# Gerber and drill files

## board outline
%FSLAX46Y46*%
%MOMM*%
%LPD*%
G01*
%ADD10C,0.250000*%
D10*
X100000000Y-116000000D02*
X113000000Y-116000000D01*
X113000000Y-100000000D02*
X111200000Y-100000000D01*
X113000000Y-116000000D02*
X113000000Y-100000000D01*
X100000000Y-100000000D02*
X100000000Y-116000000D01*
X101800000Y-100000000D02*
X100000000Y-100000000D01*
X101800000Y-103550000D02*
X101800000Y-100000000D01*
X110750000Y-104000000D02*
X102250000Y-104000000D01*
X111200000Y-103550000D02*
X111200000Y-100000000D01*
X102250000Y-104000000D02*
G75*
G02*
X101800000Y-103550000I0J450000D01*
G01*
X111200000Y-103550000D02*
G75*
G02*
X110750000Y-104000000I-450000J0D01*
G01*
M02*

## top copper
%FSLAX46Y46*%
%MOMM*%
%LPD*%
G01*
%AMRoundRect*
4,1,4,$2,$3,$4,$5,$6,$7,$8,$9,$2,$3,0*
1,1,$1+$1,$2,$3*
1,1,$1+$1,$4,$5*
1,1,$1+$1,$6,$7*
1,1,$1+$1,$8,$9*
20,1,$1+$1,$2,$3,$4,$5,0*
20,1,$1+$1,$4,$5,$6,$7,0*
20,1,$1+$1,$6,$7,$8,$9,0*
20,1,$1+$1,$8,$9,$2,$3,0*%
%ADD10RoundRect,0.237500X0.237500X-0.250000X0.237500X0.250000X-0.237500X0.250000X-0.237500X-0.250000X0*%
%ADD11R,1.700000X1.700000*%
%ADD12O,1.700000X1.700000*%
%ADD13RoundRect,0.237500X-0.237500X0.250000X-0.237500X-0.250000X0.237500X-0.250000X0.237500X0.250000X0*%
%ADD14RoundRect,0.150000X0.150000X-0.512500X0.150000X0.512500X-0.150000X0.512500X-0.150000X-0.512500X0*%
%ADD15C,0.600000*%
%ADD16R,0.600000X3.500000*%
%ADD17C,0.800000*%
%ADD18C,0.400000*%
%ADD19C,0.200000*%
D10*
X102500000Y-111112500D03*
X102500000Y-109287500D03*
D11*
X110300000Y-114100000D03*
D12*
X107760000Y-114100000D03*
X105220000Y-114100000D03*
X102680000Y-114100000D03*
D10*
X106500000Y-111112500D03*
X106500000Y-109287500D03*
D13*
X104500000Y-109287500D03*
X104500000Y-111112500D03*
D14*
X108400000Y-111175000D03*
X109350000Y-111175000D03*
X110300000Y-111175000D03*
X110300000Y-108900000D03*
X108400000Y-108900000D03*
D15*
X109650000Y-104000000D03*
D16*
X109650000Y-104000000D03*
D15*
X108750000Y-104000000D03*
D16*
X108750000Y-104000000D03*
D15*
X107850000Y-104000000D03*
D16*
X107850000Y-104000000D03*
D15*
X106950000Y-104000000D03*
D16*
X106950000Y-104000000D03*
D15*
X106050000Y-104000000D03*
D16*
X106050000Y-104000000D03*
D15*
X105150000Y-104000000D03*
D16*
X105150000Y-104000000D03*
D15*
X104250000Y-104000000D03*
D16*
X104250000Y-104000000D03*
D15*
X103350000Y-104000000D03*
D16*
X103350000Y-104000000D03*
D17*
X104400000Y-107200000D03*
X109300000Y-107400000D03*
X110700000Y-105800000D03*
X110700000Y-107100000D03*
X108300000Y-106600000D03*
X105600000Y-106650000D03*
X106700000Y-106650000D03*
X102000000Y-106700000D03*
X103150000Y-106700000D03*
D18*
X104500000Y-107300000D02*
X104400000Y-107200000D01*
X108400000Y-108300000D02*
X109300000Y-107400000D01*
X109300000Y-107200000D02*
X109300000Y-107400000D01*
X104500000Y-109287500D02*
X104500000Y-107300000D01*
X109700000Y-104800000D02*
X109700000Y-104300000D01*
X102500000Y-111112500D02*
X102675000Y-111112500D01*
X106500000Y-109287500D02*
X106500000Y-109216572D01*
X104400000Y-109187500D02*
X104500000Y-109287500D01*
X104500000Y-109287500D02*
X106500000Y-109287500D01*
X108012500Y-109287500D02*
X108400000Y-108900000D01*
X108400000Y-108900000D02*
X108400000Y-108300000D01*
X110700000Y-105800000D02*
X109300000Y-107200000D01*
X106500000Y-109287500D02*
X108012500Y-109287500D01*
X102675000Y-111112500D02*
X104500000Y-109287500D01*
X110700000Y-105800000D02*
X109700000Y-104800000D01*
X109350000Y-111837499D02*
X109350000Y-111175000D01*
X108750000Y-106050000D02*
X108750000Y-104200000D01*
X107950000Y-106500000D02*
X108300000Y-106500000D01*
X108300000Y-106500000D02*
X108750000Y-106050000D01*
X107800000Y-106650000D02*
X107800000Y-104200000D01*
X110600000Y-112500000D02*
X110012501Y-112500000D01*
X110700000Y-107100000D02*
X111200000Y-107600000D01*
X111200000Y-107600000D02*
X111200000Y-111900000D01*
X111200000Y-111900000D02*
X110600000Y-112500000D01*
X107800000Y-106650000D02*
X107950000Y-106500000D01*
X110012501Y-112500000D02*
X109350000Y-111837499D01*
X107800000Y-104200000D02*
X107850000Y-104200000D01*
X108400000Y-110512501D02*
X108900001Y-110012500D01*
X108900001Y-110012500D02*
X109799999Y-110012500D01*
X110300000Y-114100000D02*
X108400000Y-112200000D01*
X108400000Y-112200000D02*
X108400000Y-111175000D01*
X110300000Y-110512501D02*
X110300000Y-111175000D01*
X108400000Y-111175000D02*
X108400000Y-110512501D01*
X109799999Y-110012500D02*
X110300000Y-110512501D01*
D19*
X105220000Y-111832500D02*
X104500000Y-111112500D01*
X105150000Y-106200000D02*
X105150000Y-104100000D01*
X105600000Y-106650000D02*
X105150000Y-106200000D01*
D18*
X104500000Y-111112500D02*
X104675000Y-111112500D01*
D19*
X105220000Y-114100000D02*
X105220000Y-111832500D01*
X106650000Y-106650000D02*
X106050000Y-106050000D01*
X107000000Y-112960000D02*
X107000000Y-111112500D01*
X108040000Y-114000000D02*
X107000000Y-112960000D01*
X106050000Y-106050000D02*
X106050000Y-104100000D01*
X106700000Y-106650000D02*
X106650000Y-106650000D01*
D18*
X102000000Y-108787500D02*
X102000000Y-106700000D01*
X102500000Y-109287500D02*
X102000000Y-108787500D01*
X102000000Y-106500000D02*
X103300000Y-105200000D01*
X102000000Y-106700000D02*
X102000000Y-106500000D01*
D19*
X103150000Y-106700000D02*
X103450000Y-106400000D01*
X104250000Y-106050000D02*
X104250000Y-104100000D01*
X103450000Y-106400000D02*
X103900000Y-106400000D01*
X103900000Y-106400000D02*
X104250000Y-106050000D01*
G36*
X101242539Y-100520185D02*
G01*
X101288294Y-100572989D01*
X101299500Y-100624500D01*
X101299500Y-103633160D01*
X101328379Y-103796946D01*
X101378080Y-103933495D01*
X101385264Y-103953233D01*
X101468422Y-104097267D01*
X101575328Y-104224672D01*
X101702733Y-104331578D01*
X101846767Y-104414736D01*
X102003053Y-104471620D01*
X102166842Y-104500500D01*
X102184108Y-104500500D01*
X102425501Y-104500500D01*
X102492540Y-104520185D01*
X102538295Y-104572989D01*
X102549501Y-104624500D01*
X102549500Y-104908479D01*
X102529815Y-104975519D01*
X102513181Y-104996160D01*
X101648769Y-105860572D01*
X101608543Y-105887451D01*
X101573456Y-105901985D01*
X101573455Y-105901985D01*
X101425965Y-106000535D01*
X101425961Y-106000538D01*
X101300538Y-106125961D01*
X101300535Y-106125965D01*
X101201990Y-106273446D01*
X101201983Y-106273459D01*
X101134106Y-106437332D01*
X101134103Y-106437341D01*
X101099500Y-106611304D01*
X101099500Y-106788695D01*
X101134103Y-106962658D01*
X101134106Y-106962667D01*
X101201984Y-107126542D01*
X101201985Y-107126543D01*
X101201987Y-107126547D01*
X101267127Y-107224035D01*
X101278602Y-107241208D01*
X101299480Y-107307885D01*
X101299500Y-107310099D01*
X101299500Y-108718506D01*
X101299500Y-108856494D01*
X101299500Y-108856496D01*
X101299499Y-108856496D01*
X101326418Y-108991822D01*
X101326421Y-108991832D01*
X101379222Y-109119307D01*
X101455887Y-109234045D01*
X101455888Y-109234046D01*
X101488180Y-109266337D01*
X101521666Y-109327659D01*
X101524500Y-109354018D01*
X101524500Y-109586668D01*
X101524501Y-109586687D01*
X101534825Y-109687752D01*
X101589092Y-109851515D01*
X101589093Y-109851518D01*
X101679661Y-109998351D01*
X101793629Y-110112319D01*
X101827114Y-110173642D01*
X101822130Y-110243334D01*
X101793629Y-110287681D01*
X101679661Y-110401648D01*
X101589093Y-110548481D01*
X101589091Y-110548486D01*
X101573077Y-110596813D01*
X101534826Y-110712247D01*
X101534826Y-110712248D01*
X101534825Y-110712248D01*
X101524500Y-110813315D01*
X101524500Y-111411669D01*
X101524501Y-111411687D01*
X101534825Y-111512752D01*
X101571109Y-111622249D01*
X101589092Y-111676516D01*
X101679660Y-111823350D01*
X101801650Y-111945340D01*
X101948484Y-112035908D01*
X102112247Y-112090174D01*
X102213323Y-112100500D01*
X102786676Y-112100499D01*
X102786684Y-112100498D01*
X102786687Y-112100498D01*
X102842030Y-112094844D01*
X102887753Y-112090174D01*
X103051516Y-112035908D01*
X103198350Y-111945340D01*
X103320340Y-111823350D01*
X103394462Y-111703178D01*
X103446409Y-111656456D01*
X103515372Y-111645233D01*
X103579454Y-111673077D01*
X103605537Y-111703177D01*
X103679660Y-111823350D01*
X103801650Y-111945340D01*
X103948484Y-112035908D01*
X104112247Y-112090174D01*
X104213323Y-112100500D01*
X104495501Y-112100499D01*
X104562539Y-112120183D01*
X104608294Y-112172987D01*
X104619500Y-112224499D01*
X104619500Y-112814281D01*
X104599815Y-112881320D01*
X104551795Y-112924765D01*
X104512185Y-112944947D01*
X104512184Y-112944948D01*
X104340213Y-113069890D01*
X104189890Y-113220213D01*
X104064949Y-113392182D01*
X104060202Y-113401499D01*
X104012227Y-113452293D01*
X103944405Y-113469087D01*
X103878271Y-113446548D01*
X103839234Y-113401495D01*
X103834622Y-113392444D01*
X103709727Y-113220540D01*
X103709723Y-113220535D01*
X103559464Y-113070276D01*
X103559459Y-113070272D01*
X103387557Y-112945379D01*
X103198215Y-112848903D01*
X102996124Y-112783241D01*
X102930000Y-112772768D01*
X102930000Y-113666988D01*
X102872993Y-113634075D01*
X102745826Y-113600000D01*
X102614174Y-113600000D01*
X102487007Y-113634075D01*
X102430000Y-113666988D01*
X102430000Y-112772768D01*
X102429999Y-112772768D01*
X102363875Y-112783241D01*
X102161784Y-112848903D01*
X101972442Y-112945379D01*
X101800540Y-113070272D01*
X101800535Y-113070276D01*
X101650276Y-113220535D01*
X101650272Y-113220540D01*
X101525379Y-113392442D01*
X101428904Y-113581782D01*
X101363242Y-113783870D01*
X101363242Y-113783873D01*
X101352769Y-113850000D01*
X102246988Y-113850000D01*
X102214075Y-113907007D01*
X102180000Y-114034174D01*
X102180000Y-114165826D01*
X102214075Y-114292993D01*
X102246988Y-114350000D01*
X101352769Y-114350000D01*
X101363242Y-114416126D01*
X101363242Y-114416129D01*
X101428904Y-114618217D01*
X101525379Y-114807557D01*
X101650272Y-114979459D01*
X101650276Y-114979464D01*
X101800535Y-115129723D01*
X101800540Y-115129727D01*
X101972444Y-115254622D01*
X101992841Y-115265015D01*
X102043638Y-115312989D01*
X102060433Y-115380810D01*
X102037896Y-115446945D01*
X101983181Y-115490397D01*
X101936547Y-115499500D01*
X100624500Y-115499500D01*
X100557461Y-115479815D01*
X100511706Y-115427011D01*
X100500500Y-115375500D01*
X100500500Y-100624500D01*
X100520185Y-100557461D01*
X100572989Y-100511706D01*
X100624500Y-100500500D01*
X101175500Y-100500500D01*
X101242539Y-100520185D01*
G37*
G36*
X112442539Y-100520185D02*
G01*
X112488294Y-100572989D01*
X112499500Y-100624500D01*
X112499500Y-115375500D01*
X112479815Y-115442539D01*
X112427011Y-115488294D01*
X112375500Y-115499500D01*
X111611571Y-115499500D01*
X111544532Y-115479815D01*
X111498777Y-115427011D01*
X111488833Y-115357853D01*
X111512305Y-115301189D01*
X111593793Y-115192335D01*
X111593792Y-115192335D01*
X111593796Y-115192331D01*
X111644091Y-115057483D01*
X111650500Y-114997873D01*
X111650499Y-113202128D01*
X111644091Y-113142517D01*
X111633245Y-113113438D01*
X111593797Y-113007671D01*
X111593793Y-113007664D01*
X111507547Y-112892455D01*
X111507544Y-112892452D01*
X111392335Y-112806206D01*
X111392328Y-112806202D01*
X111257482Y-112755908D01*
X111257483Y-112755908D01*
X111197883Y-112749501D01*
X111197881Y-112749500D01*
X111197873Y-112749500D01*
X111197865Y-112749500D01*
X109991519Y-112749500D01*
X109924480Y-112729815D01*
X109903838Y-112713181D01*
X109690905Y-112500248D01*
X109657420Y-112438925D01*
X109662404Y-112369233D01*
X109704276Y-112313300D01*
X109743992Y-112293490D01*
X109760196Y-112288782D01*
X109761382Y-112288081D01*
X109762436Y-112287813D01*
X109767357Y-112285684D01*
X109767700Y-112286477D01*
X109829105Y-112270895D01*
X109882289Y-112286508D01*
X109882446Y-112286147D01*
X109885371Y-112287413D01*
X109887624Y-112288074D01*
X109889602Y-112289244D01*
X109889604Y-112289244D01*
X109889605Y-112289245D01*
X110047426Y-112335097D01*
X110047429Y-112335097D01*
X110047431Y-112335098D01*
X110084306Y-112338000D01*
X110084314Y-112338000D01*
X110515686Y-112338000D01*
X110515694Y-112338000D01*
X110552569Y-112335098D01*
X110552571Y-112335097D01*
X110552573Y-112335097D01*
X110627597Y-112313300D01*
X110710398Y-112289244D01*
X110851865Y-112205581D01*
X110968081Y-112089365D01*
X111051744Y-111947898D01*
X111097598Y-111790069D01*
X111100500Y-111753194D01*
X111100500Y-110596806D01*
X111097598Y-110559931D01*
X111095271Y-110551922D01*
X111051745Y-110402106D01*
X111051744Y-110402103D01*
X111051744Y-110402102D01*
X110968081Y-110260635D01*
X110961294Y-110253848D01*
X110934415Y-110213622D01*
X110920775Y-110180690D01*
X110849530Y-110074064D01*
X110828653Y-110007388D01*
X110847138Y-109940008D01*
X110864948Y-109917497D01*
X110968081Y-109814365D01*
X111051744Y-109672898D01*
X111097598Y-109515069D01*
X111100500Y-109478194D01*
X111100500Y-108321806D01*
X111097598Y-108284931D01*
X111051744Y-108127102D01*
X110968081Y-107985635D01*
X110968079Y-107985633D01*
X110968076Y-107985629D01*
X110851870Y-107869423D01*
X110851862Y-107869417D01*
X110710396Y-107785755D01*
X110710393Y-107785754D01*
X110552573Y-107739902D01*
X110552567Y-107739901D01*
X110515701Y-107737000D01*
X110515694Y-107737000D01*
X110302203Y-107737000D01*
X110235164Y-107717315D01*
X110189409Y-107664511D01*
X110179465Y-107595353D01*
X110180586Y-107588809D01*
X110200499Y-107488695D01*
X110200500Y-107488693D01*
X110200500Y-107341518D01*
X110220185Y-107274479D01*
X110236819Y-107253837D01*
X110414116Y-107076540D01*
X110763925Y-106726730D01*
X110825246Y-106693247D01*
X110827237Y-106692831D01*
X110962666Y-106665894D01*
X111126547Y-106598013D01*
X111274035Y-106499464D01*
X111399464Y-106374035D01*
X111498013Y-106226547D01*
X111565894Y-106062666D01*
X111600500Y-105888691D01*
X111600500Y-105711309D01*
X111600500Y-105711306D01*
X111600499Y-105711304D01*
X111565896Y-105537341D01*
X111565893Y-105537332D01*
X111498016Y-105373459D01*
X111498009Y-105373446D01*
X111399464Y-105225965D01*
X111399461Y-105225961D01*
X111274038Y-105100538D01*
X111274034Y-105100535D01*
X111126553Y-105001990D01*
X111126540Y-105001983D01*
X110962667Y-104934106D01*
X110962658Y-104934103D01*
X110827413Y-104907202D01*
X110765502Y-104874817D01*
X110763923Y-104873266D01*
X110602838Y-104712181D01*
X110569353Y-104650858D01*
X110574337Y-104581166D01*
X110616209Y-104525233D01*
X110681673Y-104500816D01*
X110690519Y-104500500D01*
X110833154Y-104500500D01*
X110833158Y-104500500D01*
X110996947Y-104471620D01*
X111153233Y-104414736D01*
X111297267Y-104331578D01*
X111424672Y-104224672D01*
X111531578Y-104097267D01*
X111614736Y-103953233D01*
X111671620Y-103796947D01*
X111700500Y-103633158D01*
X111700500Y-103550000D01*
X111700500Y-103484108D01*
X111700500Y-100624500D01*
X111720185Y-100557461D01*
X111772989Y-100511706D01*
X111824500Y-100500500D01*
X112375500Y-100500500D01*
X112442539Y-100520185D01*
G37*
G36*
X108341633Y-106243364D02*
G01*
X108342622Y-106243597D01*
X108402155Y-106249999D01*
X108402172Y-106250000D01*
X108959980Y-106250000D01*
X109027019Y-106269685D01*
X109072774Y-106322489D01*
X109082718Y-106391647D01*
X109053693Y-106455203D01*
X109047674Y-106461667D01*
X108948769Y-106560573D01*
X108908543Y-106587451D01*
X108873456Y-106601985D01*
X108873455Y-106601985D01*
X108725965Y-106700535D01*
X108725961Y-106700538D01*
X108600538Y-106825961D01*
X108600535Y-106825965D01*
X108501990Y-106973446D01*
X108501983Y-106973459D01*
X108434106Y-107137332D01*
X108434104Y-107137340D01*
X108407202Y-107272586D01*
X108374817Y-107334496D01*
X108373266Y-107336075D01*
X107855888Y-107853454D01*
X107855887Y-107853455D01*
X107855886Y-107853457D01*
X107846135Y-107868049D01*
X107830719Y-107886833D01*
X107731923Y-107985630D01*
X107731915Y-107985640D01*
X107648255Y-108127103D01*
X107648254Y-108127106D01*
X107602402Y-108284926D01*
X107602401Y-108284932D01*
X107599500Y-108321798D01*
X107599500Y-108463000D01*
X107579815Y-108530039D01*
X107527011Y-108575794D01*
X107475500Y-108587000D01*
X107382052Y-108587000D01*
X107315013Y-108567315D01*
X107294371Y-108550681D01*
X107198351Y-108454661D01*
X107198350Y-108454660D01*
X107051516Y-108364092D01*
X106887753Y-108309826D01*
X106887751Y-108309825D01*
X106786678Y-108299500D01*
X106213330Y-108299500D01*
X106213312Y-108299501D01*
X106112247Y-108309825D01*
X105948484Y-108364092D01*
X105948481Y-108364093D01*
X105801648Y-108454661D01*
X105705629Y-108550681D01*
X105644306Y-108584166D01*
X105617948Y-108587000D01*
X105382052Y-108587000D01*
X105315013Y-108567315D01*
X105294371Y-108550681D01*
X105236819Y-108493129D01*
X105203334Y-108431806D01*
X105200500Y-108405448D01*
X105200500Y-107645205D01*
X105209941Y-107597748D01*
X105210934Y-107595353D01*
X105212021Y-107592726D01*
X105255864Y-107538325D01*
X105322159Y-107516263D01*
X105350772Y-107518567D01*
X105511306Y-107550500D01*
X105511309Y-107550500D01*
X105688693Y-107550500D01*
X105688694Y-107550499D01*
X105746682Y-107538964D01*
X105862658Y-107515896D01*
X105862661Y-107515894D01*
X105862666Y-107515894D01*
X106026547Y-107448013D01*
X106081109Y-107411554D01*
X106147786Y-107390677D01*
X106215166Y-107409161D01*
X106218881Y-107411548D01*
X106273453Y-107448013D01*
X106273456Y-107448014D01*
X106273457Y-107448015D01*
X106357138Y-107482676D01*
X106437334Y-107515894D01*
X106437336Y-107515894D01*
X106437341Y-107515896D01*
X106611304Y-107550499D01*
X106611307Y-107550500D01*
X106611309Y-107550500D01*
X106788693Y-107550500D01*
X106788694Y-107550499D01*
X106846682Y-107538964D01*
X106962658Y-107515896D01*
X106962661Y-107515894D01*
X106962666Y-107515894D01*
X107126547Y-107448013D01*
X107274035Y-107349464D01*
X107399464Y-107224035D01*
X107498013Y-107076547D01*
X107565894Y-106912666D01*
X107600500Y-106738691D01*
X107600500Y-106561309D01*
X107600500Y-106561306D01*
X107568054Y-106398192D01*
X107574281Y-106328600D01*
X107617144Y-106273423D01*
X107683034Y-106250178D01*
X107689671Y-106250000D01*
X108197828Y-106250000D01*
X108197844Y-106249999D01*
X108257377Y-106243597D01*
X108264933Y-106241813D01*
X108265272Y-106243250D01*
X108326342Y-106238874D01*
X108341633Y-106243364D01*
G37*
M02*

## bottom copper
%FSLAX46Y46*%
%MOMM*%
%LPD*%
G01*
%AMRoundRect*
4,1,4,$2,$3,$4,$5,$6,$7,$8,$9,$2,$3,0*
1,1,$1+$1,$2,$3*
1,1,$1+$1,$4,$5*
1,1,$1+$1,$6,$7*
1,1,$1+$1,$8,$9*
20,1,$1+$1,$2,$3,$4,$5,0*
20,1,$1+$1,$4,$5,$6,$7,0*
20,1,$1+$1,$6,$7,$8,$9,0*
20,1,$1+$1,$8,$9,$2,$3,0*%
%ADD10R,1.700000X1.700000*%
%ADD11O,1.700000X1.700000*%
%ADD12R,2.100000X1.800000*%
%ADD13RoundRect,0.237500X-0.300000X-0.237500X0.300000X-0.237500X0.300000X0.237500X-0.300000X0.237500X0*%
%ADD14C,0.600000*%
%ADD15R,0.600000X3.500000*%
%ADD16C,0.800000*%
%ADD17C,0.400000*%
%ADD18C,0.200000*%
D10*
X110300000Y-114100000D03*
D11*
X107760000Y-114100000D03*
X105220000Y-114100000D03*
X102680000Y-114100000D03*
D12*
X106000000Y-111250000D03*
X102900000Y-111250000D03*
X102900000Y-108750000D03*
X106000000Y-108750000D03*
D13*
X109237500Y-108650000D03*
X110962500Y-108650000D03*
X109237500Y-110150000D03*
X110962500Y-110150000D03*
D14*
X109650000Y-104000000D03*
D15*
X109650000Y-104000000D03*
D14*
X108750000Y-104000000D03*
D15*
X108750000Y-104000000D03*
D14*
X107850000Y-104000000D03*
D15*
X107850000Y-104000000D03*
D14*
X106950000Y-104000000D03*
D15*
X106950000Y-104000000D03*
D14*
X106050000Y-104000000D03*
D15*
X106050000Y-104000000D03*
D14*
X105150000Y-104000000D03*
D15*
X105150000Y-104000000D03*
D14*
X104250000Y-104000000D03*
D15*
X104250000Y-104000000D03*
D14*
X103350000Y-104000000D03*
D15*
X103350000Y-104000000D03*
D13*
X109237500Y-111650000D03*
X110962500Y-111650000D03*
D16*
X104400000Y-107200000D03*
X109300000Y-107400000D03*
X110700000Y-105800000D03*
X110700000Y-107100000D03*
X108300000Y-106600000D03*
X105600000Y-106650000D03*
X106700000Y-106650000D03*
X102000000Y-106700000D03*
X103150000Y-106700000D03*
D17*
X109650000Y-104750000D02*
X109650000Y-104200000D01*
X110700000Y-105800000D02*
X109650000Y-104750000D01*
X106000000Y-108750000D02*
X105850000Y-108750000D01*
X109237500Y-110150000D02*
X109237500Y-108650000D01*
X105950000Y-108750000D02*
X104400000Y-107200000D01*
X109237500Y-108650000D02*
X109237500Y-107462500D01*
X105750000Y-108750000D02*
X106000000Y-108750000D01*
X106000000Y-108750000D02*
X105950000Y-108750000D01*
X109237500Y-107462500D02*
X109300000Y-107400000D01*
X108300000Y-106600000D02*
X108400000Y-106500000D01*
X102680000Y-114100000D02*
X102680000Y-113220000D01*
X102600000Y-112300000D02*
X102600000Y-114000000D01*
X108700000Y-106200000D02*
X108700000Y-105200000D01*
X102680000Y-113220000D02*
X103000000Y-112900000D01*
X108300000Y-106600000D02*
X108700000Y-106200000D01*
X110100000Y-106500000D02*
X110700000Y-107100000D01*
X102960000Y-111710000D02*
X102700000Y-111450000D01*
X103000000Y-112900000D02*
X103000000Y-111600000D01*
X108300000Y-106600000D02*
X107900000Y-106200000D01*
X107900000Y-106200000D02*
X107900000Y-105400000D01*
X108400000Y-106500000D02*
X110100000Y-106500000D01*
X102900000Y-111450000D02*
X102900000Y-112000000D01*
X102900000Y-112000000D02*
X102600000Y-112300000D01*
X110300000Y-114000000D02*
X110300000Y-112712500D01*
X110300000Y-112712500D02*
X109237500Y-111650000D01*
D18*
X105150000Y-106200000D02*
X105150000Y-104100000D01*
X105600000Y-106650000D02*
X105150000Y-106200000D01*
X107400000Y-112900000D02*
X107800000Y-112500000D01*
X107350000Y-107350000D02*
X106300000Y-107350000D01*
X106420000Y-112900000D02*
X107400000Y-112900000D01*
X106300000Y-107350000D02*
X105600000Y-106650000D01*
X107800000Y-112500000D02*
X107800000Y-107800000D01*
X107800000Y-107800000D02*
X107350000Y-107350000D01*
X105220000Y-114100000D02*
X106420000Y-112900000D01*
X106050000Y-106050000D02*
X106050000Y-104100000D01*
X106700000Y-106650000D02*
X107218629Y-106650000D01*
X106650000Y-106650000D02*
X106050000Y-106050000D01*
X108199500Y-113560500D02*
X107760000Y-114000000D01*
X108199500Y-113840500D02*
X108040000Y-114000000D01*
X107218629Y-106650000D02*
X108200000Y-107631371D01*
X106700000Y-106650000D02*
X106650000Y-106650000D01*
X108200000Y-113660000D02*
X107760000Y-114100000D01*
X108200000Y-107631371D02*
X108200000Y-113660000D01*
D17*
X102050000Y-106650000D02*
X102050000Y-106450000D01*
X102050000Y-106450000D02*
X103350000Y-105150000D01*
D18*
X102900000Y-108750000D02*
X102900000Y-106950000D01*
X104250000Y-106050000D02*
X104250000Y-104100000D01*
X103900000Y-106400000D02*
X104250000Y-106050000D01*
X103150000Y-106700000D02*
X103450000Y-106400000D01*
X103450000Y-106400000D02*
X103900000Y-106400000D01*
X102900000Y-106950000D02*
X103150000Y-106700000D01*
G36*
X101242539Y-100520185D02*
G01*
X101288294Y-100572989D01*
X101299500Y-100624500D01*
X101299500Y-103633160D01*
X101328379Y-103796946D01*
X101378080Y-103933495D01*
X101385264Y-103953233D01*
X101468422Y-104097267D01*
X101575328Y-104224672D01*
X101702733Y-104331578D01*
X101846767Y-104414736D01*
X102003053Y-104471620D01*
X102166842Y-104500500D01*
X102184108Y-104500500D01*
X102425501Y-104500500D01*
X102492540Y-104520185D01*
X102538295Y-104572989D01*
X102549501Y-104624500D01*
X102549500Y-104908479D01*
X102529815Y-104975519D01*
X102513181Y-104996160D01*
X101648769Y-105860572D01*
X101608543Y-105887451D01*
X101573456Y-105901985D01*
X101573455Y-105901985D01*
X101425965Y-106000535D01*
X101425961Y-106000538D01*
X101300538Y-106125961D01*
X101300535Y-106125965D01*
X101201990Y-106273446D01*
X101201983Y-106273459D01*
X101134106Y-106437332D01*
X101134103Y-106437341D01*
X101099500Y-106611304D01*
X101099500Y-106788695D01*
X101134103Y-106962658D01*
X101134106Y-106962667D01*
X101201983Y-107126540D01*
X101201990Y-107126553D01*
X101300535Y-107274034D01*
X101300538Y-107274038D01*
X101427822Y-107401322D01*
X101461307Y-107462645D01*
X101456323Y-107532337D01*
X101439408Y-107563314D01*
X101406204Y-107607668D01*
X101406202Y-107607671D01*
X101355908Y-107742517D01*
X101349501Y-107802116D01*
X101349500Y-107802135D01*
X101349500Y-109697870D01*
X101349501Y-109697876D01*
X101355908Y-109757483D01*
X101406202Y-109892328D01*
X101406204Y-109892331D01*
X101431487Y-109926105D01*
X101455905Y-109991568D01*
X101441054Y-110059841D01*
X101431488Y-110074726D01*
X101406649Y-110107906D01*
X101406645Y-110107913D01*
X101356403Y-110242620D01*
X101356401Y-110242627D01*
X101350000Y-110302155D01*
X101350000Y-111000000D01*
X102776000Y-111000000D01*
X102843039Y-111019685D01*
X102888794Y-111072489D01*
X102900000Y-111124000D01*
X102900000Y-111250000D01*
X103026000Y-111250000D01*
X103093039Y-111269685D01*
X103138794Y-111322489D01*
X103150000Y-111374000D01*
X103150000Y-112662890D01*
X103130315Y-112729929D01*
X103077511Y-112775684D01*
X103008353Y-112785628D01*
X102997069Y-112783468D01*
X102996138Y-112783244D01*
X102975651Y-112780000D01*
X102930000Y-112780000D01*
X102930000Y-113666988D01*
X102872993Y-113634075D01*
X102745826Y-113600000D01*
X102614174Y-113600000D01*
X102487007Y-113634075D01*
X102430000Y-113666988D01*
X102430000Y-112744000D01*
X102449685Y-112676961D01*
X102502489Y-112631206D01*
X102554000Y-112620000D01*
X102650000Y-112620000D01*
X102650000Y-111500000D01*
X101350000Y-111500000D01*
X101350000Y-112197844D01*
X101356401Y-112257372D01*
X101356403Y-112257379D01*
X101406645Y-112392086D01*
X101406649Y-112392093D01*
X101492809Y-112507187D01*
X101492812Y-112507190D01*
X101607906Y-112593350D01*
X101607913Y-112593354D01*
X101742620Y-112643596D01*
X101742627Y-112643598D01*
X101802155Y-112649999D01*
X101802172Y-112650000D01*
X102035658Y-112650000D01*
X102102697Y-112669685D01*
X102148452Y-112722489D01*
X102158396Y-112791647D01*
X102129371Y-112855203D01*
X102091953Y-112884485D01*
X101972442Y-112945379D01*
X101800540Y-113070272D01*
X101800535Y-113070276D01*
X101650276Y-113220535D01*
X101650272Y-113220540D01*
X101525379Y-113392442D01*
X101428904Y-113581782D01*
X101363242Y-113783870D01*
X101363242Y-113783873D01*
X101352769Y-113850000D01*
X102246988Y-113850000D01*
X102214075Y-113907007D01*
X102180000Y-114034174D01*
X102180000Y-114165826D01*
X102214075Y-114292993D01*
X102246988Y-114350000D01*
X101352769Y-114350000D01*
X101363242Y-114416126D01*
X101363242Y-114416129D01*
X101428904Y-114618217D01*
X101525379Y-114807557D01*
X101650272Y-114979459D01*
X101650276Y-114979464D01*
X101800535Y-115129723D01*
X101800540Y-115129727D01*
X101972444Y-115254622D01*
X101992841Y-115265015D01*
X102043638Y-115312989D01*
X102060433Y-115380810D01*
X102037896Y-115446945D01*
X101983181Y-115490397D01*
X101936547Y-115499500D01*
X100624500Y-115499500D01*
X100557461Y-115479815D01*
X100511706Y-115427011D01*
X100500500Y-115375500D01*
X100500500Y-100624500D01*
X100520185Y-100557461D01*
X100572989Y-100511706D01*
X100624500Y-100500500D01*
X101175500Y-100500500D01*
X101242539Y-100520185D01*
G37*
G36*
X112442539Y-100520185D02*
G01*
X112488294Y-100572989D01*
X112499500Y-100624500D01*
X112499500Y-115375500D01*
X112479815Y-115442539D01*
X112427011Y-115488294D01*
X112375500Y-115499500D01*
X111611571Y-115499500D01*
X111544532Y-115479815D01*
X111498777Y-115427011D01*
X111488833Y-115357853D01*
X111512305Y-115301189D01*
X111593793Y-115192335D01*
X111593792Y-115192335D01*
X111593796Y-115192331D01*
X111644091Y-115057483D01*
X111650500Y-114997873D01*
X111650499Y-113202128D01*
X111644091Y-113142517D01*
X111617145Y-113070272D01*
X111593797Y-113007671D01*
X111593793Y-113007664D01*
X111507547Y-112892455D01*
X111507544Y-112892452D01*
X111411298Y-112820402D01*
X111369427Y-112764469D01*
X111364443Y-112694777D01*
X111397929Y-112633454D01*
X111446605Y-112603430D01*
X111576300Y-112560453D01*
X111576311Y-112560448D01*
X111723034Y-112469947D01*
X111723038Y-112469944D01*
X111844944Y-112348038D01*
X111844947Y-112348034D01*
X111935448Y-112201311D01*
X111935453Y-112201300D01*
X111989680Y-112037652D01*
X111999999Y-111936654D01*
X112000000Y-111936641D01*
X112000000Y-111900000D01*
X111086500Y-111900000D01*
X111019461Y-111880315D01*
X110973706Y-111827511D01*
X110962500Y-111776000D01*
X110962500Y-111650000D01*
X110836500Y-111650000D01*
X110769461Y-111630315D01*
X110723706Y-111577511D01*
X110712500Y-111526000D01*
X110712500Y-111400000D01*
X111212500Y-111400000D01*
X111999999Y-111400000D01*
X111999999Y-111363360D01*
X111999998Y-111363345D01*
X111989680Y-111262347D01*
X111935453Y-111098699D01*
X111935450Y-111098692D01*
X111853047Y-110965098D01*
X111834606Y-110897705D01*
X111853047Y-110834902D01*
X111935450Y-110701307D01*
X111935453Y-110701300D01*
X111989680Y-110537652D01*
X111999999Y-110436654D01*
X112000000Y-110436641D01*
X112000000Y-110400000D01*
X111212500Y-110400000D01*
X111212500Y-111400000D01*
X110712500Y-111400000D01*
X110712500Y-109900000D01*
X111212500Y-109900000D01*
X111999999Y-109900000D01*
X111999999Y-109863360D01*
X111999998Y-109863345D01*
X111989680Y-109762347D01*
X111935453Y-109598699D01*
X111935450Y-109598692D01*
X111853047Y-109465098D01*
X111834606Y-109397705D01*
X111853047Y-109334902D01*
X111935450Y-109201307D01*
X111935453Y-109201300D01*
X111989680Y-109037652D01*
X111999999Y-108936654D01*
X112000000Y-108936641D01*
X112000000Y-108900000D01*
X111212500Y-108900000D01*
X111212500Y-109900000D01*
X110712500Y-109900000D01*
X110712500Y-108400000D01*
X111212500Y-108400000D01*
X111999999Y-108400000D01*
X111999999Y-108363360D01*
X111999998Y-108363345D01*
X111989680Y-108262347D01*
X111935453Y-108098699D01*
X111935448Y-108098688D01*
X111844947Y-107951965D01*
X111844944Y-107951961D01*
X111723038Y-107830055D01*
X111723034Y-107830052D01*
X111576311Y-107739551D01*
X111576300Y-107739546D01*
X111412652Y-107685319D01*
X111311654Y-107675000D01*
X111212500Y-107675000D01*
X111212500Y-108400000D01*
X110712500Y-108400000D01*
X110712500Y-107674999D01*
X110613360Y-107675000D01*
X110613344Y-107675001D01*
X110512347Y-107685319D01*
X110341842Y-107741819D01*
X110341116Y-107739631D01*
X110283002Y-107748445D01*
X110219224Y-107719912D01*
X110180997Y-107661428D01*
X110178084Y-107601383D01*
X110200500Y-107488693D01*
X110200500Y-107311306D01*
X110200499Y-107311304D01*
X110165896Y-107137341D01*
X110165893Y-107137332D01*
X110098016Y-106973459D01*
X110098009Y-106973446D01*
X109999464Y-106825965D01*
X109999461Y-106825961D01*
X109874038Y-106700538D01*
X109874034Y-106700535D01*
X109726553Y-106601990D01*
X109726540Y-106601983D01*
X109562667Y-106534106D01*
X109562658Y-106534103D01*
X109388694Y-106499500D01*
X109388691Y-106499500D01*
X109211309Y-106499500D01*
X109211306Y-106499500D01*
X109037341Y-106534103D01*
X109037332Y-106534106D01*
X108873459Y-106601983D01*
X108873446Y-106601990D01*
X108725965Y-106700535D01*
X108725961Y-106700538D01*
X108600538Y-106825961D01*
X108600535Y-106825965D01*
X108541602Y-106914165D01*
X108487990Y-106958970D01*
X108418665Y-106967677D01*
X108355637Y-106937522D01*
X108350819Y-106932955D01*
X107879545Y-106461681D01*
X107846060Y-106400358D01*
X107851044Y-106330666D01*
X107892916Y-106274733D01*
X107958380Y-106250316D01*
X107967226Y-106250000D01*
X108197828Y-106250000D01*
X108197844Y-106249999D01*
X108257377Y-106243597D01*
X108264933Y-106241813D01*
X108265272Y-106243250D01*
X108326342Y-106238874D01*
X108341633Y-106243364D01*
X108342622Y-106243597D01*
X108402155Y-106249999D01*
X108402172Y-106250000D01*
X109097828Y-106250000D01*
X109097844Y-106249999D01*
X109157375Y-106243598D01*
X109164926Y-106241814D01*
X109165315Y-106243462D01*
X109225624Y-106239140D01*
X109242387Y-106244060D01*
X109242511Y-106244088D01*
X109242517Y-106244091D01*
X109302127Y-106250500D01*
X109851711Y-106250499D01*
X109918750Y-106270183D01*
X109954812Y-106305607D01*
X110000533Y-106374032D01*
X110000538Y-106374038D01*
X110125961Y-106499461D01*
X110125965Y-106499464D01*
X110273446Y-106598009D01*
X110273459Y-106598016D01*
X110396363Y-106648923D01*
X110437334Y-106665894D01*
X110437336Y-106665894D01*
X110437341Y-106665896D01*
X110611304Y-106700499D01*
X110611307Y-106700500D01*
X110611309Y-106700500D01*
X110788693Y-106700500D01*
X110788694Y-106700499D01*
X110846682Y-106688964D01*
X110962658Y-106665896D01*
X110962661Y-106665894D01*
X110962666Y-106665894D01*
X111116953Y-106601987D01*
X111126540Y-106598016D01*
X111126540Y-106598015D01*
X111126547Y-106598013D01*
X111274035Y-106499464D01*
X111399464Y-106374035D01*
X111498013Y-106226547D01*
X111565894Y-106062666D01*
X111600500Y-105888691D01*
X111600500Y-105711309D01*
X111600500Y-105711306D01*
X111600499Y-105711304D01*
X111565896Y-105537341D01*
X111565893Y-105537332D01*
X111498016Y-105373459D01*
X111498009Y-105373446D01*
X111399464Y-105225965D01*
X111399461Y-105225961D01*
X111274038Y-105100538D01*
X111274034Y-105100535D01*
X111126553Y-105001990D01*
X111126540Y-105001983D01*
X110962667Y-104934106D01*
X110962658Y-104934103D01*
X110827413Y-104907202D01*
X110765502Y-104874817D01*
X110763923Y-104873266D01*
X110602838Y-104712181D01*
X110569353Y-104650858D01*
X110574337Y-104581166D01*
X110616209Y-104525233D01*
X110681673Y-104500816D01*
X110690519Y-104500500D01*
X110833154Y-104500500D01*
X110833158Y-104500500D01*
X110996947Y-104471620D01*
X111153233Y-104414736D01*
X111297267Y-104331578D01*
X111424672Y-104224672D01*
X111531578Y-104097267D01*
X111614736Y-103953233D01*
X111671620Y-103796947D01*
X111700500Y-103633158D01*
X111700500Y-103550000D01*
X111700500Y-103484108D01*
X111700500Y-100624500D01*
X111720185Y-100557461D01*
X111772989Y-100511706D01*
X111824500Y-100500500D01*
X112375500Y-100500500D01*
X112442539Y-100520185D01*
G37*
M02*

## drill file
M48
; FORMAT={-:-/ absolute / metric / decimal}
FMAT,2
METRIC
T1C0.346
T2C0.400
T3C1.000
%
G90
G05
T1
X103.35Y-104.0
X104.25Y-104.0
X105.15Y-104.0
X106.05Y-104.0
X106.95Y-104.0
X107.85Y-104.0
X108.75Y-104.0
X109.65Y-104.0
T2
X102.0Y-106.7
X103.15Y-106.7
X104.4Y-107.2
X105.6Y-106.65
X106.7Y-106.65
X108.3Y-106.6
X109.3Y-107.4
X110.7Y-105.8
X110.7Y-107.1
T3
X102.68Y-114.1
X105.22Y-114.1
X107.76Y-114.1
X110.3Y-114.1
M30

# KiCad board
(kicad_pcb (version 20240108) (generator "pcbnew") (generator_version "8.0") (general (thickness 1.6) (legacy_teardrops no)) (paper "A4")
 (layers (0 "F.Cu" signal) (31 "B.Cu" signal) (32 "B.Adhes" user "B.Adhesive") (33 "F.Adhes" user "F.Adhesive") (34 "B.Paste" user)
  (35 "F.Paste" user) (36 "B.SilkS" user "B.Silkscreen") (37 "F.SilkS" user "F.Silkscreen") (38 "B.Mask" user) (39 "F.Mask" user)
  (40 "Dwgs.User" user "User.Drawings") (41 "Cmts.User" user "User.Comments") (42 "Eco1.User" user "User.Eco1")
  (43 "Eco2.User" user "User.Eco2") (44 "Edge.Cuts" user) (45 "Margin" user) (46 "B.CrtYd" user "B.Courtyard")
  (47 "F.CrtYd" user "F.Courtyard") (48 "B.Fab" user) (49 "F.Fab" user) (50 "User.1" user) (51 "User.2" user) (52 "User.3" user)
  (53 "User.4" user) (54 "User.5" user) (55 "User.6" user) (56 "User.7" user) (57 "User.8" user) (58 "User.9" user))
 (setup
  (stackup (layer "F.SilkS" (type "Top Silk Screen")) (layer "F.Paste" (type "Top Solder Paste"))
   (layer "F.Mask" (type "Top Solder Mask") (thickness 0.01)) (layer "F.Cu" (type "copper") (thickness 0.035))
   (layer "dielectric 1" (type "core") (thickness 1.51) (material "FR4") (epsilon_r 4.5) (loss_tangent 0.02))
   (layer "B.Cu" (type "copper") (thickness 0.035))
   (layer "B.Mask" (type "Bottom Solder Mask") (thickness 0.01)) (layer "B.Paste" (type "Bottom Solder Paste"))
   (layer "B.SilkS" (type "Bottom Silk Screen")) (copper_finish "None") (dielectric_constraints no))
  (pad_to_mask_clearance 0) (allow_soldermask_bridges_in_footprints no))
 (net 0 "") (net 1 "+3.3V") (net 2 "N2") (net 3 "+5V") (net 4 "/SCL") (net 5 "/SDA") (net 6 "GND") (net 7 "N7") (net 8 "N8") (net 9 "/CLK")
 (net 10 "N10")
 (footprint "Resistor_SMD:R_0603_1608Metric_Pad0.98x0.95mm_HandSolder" (layer "F.Cu") (at 102.5 110.2 90)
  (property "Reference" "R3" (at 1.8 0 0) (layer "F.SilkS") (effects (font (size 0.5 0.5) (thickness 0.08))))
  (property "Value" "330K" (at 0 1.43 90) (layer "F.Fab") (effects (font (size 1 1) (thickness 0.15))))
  (pad "1" smd roundrect (at -0.9125 0 90) (size 0.975 0.95) (layers "F.Cu" "F.Paste" "F.Mask") (roundrect_rratio 0.25) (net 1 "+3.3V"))
  (pad "2" smd roundrect (at 0.9125 0 90) (size 0.975 0.95) (layers "F.Cu" "F.Paste" "F.Mask") (roundrect_rratio 0.25) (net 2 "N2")))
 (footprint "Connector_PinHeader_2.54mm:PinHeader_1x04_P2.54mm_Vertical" (layer "F.Cu") (at 110.3 114.1 -90)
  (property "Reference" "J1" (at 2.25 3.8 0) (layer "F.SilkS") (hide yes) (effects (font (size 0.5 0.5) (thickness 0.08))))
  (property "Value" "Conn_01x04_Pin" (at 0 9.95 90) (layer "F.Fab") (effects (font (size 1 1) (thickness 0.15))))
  (pad "1" thru_hole rect (at 0 0 270) (size 1.7 1.7) (drill 1) (layers "*.Cu" "*.Mask") (remove_unused_layers no) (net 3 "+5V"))
  (pad "2" thru_hole oval (at 0 2.54 270) (size 1.7 1.7) (drill 1) (layers "*.Cu" "*.Mask") (remove_unused_layers no) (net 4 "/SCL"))
  (pad "3" thru_hole oval (at 0 5.08 270) (size 1.7 1.7) (drill 1) (layers "*.Cu" "*.Mask") (remove_unused_layers no) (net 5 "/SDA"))
  (pad "4" thru_hole oval (at 0 7.62 270) (size 1.7 1.7) (drill 1) (layers "*.Cu" "*.Mask") (remove_unused_layers no) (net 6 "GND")))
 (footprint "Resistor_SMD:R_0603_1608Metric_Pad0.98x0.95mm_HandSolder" (layer "F.Cu") (at 106.5 110.2 90)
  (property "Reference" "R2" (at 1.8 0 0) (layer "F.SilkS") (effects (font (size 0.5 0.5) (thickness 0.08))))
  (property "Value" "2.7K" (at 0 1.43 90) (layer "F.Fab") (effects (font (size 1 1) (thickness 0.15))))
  (pad "1" smd roundrect (at -0.9125 0 90) (size 0.975 0.95) (layers "F.Cu" "F.Paste" "F.Mask") (roundrect_rratio 0.25) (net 4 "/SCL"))
  (pad "2" smd roundrect (at 0.9125 0 90) (size 0.975 0.95) (layers "F.Cu" "F.Paste" "F.Mask") (roundrect_rratio 0.25) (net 1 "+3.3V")))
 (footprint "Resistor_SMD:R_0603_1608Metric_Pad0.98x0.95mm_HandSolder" (layer "F.Cu") (at 104.5 110.2 -90)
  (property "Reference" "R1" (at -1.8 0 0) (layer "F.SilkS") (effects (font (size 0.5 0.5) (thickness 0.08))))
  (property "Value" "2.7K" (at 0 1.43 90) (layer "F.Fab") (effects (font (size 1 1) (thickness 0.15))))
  (pad "1" smd roundrect (at -0.9125 0 270) (size 0.975 0.95) (layers "F.Cu" "F.Paste" "F.Mask") (roundrect_rratio 0.25) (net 1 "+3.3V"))
  (pad "2" smd roundrect (at 0.9125 0 270) (size 0.975 0.95) (layers "F.Cu" "F.Paste" "F.Mask") (roundrect_rratio 0.25) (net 5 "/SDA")))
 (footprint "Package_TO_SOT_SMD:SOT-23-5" (layer "F.Cu") (at 109.35 110.0375 90)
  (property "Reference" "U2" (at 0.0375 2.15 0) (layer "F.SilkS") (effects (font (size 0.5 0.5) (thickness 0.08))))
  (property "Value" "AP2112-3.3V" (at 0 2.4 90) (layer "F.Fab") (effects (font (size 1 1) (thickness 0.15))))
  (pad "1" smd roundrect (at -1.1375 -0.95 90) (size 1.325 0.6) (layers "F.Cu" "F.Paste" "F.Mask") (roundrect_rratio 0.25) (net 3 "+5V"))
  (pad "2" smd roundrect (at -1.1375 0 90) (size 1.325 0.6) (layers "F.Cu" "F.Paste" "F.Mask") (roundrect_rratio 0.25) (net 6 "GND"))
  (pad "3" smd roundrect (at -1.1375 0.95 90) (size 1.325 0.6) (layers "F.Cu" "F.Paste" "F.Mask") (roundrect_rratio 0.25) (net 3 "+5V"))
  (pad "4" smd roundrect (at 1.1375 0.95 90) (size 1.325 0.6) (layers "F.Cu" "F.Paste" "F.Mask") (roundrect_rratio 0.25) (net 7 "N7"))
  (pad "5" smd roundrect (at 1.1375 -0.95 90) (size 1.325 0.6) (layers "F.Cu" "F.Paste" "F.Mask") (roundrect_rratio 0.25) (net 1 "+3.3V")))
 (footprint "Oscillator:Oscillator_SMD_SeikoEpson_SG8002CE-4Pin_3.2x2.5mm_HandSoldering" (layer "B.Cu") (at 104.45 110 180)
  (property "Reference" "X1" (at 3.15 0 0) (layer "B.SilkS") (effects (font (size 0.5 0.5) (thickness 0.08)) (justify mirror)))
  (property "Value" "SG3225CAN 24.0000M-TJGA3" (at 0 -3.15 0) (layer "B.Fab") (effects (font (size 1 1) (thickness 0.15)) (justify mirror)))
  (pad "1" smd rect (at -1.55 -1.25 180) (size 2.1 1.8) (layers "B.Cu" "B.Paste" "B.Mask") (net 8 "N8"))
  (pad "2" smd rect (at 1.55 -1.25 180) (size 2.1 1.8) (layers "B.Cu" "B.Paste" "B.Mask") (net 6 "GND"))
  (pad "3" smd rect (at 1.55 1.25 180) (size 2.1 1.8) (layers "B.Cu" "B.Paste" "B.Mask") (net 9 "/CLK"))
  (pad "4" smd rect (at -1.55 1.25 180) (size 2.1 1.8) (layers "B.Cu" "B.Paste" "B.Mask") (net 1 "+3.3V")))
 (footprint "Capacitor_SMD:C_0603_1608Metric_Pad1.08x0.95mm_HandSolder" (layer "B.Cu") (at 110.1 108.65)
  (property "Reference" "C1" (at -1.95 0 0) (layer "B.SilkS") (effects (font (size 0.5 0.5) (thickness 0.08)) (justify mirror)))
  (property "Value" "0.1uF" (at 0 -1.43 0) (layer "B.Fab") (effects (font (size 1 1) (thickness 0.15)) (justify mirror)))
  (pad "1" smd roundrect (at -0.8625 0) (size 1.075 0.95) (layers "B.Cu" "B.Paste" "B.Mask") (roundrect_rratio 0.25) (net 1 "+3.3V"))
  (pad "2" smd roundrect (at 0.8625 0) (size 1.075 0.95) (layers "B.Cu" "B.Paste" "B.Mask") (roundrect_rratio 0.25) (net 6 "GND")))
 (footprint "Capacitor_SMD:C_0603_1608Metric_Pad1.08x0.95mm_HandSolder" (layer "B.Cu") (at 110.1 110.15)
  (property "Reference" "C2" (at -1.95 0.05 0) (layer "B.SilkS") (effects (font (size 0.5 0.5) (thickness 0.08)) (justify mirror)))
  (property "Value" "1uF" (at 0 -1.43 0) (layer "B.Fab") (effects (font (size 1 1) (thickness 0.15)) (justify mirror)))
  (pad "1" smd roundrect (at -0.8625 0) (size 1.075 0.95) (layers "B.Cu" "B.Paste" "B.Mask") (roundrect_rratio 0.25) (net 1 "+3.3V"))
  (pad "2" smd roundrect (at 0.8625 0) (size 1.075 0.95) (layers "B.Cu" "B.Paste" "B.Mask") (roundrect_rratio 0.25) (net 6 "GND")))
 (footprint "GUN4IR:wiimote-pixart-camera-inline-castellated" (layer "B.Cu") (at 106.5 101.5 180)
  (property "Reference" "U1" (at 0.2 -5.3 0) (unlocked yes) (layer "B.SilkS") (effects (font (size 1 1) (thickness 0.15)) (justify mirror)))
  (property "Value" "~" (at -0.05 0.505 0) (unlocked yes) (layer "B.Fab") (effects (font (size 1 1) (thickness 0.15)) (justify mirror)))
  (fp_line (start 4.7 -2.05) (end 4.7 1.5) (stroke (width 0.25) (type default)) (layer "Edge.Cuts"))
  (fp_line (start -4.25 -2.5) (end 4.25 -2.5) (stroke (width 0.25) (type default)) (layer "Edge.Cuts"))
  (fp_line (start -4.7 -2.05) (end -4.7 1.5) (stroke (width 0.25) (type default)) (layer "Edge.Cuts"))
  (fp_arc (start 4.25 -2.5) (mid 4.568198 -2.368198) (end 4.7 -2.05) (stroke (width 0.25) (type default)) (layer "Edge.Cuts"))
  (fp_arc (start -4.7 -2.05) (mid -4.568198 -2.368198) (end -4.25 -2.5) (stroke (width 0.25) (type default)) (layer "Edge.Cuts"))
  (pad "1" thru_hole circle (at -3.15 -2.5 180) (size 0.6 0.6) (drill 0.346) (layers "*.Cu" "*.Mask") (remove_unused_layers no)
   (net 1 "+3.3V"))
  (pad "1" smd rect (at -3.15 -2.5 180) (size 0.6 3.5) (layers "F.Cu" "F.Paste" "F.Mask") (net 1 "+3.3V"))
  (pad "1" smd rect (at -3.15 -2.5 180) (size 0.6 3.5) (layers "B.Cu" "B.Paste" "B.Mask") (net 1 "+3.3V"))
  (pad "2" thru_hole circle (at -2.25 -2.5 180) (size 0.6 0.6) (drill 0.346) (layers "*.Cu" "*.Mask") (remove_unused_layers no)
   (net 6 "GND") (zone_connect 0))
  (pad "2" smd rect (at -2.25 -2.5 180) (size 0.6 3.5) (layers "F.Cu" "F.Paste" "F.Mask") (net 6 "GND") (zone_connect 0))
  (pad "2" smd rect (at -2.25 -2.5 180) (size 0.6 3.5) (layers "B.Cu" "B.Paste" "B.Mask") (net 6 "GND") (zone_connect 0))
  (pad "3" thru_hole circle (at -1.35 -2.5 180) (size 0.6 0.6) (drill 0.346) (layers "*.Cu" "*.Mask") (remove_unused_layers no)
   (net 6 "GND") (zone_connect 0))
  (pad "3" smd rect (at -1.35 -2.5 180) (size 0.6 3.5) (layers "F.Cu" "F.Paste" "F.Mask") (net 6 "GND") (zone_connect 0))
  (pad "3" smd rect (at -1.35 -2.5 180) (size 0.6 3.5) (layers "B.Cu" "B.Paste" "B.Mask") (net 6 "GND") (zone_connect 0))
  (pad "4" thru_hole circle (at -0.45 -2.5 180) (size 0.6 0.6) (drill 0.346) (layers "*.Cu" "*.Mask") (remove_unused_layers no)
   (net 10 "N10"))
  (pad "4" smd rect (at -0.45 -2.5 180) (size 0.6 3.5) (layers "F.Cu" "F.Paste" "F.Mask") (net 10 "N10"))
  (pad "4" smd rect (at -0.45 -2.5 180) (size 0.6 3.5) (layers "B.Cu" "B.Paste" "B.Mask") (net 10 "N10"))
  (pad "5" thru_hole circle (at 0.45 -2.5 180) (size 0.6 0.6) (drill 0.346) (layers "*.Cu" "*.Mask") (remove_unused_layers no)
   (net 4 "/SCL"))
  (pad "5" smd rect (at 0.45 -2.5 180) (size 0.6 3.5) (layers "F.Cu" "F.Paste" "F.Mask") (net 4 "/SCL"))
  (pad "5" smd rect (at 0.45 -2.5 180) (size 0.6 3.5) (layers "B.Cu" "B.Paste" "B.Mask") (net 4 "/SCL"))
  (pad "6" thru_hole circle (at 1.35 -2.5 180) (size 0.6 0.6) (drill 0.346) (layers "*.Cu" "*.Mask") (remove_unused_layers no)
   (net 5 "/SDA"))
  (pad "6" smd rect (at 1.35 -2.5 180) (size 0.6 3.5) (layers "F.Cu" "F.Paste" "F.Mask") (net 5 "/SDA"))
  (pad "6" smd rect (at 1.35 -2.5 180) (size 0.6 3.5) (layers "B.Cu" "B.Paste" "B.Mask") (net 5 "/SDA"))
  (pad "7" thru_hole circle (at 2.25 -2.5 180) (size 0.6 0.6) (drill 0.346) (layers "*.Cu" "*.Mask") (remove_unused_layers no)
   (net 9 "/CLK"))
  (pad "7" smd rect (at 2.25 -2.5 180) (size 0.6 3.5) (layers "F.Cu" "F.Paste" "F.Mask") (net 9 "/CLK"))
  (pad "7" smd rect (at 2.25 -2.5 180) (size 0.6 3.5) (layers "B.Cu" "B.Paste" "B.Mask") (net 9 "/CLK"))
  (pad "8" thru_hole circle (at 3.15 -2.5 180) (size 0.6 0.6) (drill 0.346) (layers "*.Cu" "*.Mask") (remove_unused_layers no) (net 2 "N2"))
  (pad "8" smd rect (at 3.15 -2.5 180) (size 0.6 3.5) (layers "F.Cu" "F.Paste" "F.Mask") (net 2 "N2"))
  (pad "8" smd rect (at 3.15 -2.5 180) (size 0.6 3.5) (layers "B.Cu" "B.Paste" "B.Mask") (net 2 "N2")))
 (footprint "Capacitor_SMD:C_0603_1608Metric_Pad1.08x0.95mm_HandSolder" (layer "B.Cu") (at 110.1 111.65)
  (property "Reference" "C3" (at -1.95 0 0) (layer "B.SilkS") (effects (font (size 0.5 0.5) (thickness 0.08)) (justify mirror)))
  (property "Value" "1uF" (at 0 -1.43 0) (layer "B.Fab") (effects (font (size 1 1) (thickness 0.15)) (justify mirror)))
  (pad "1" smd roundrect (at -0.8625 0) (size 1.075 0.95) (layers "B.Cu" "B.Paste" "B.Mask") (roundrect_rratio 0.25) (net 3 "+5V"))
  (pad "2" smd roundrect (at 0.8625 0) (size 1.075 0.95) (layers "B.Cu" "B.Paste" "B.Mask") (roundrect_rratio 0.25) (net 6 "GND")))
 (gr_line (start 100 116) (end 113 116) (stroke (width 0.25) (type default)) (layer "Edge.Cuts"))
 (gr_line (start 113 100) (end 111.2 100) (stroke (width 0.25) (type default)) (layer "Edge.Cuts"))
 (gr_line (start 113 116) (end 113 100) (stroke (width 0.25) (type default)) (layer "Edge.Cuts"))
 (gr_line (start 100 100) (end 100 116) (stroke (width 0.25) (type default)) (layer "Edge.Cuts"))
 (gr_line (start 101.8 100) (end 100 100) (stroke (width 0.25) (type default)) (layer "Edge.Cuts"))
 (segment (start 104.5 107.3) (end 104.4 107.2) (width 0.4) (layer "F.Cu") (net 1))
 (segment (start 108.4 108.3) (end 109.3 107.4) (width 0.4) (layer "F.Cu") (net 1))
 (segment (start 109.3 107.2) (end 109.3 107.4) (width 0.4) (layer "F.Cu") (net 1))
 (segment (start 104.5 109.2875) (end 104.5 107.3) (width 0.4) (layer "F.Cu") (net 1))
 (segment (start 109.7 104.8) (end 109.7 104.3) (width 0.4) (layer "F.Cu") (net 1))
 (segment (start 102.5 111.1125) (end 102.675 111.1125) (width 0.4) (layer "F.Cu") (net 1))
 (segment (start 106.5 109.2875) (end 106.5 109.216572) (width 0.4) (layer "F.Cu") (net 1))
 (segment (start 104.4 109.1875) (end 104.5 109.2875) (width 0.4) (layer "F.Cu") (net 1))
 (segment (start 104.5 109.2875) (end 106.5 109.2875) (width 0.4) (layer "F.Cu") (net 1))
 (segment (start 108.0125 109.2875) (end 108.4 108.9) (width 0.4) (layer "F.Cu") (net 1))
 (segment (start 108.4 108.9) (end 108.4 108.3) (width 0.4) (layer "F.Cu") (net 1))
 (segment (start 110.7 105.8) (end 109.3 107.2) (width 0.4) (layer "F.Cu") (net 1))
 (segment (start 106.5 109.2875) (end 108.0125 109.2875) (width 0.4) (layer "F.Cu") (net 1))
 (segment (start 102.675 111.1125) (end 104.5 109.2875) (width 0.4) (layer "F.Cu") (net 1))
 (segment (start 110.7 105.8) (end 109.7 104.8) (width 0.4) (layer "F.Cu") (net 1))
 (via (at 104.4 107.2) (size 0.8) (drill 0.4) (layers "F.Cu" "B.Cu") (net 1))
 (via (at 109.3 107.4) (size 0.8) (drill 0.4) (layers "F.Cu" "B.Cu") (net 1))
 (via (at 110.7 105.8) (size 0.8) (drill 0.4) (layers "F.Cu" "B.Cu") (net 1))
 (segment (start 109.65 104.75) (end 109.65 104.2) (width 0.4) (layer "B.Cu") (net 1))
 (segment (start 110.7 105.8) (end 109.65 104.75) (width 0.4) (layer "B.Cu") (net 1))
 (segment (start 106 108.75) (end 105.85 108.75) (width 0.4) (layer "B.Cu") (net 1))
 (segment (start 109.2375 110.15) (end 109.2375 108.65) (width 0.4) (layer "B.Cu") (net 1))
 (segment (start 105.95 108.75) (end 104.4 107.2) (width 0.4) (layer "B.Cu") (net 1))
 (segment (start 109.2375 108.65) (end 109.2375 107.4625) (width 0.4) (layer "B.Cu") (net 1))
 (segment (start 105.75 108.75) (end 106 108.75) (width 0.4) (layer "B.Cu") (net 1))
 (segment (start 106 108.75) (end 105.95 108.75) (width 0.4) (layer "B.Cu") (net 1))
 (segment (start 109.2375 107.4625) (end 109.3 107.4) (width 0.4) (layer "B.Cu") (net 1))
 (segment (start 109.35 111.837499) (end 109.35 111.175) (width 0.4) (layer "F.Cu") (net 6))
 (segment (start 108.75 106.05) (end 108.75 104.2) (width 0.4) (layer "F.Cu") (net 6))
 (segment (start 107.95 106.5) (end 108.3 106.5) (width 0.4) (layer "F.Cu") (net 6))
 (segment (start 108.3 106.5) (end 108.75 106.05) (width 0.4) (layer "F.Cu") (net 6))
 (segment (start 107.8 106.65) (end 107.8 104.2) (width 0.4) (layer "F.Cu") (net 6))
 (segment (start 110.6 112.5) (end 110.012501 112.5) (width 0.4) (layer "F.Cu") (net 6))
 (segment (start 110.7 107.1) (end 111.2 107.6) (width 0.4) (layer "F.Cu") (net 6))
 (segment (start 111.2 107.6) (end 111.2 111.9) (width 0.4) (layer "F.Cu") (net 6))
 (segment (start 111.2 111.9) (end 110.6 112.5) (width 0.4) (layer "F.Cu") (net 6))
 (segment (start 107.8 106.65) (end 107.95 106.5) (width 0.4) (layer "F.Cu") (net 6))
 (segment (start 110.012501 112.5) (end 109.35 111.837499) (width 0.4) (layer "F.Cu") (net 6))
 (segment (start 107.8 104.2) (end 107.85 104.2) (width 0.4) (layer "F.Cu") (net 6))
 (via (at 110.7 107.1) (size 0.8) (drill 0.4) (layers "F.Cu" "B.Cu") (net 6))
 (via (at 108.3 106.6) (size 0.8) (drill 0.4) (layers "F.Cu" "B.Cu") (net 6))
 (segment (start 108.3 106.6) (end 108.4 106.5) (width 0.4) (layer "B.Cu") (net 6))
 (segment (start 102.68 114.1) (end 102.68 113.22) (width 0.4) (layer "B.Cu") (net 6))
 (segment (start 102.6 112.3) (end 102.6 114) (width 0.4) (layer "B.Cu") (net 6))
 (segment (start 108.7 106.2) (end 108.7 105.2) (width 0.4) (layer "B.Cu") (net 6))
 (segment (start 102.68 113.22) (end 103 112.9) (width 0.4) (layer "B.Cu") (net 6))
 (segment (start 108.3 106.6) (end 108.7 106.2) (width 0.4) (layer "B.Cu") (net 6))
 (segment (start 110.1 106.5) (end 110.7 107.1) (width 0.4) (layer "B.Cu") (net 6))
 (segment (start 102.96 111.71) (end 102.7 111.45) (width 0.4) (layer "B.Cu") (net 6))
 (segment (start 103 112.9) (end 103 111.6) (width 0.4) (layer "B.Cu") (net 6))
 (segment (start 108.3 106.6) (end 107.9 106.2) (width 0.4) (layer "B.Cu") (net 6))
 (segment (start 107.9 106.2) (end 107.9 105.4) (width 0.4) (layer "B.Cu") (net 6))
 (segment (start 108.4 106.5) (end 110.1 106.5) (width 0.4) (layer "B.Cu") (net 6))
 (segment (start 102.9 111.45) (end 102.9 112) (width 0.4) (layer "B.Cu") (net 6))
 (segment (start 102.9 112) (end 102.6 112.3) (width 0.4) (layer "B.Cu") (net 6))
 (segment (start 108.4 110.512501) (end 108.900001 110.0125) (width 0.4) (layer "F.Cu") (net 3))
 (segment (start 108.900001 110.0125) (end 109.799999 110.0125) (width 0.4) (layer "F.Cu") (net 3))
 (segment (start 110.3 114.1) (end 108.4 112.2) (width 0.4) (layer "F.Cu") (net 3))
 (segment (start 108.4 112.2) (end 108.4 111.175) (width 0.4) (layer "F.Cu") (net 3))
 (segment (start 110.3 110.512501) (end 110.3 111.175) (width 0.4) (layer "F.Cu") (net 3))
 (segment (start 108.4 111.175) (end 108.4 110.512501) (width 0.4) (layer "F.Cu") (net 3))
 (segment (start 109.799999 110.0125) (end 110.3 110.512501) (width 0.4) (layer "F.Cu") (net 3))
 (segment (start 110.3 114) (end 110.3 112.7125) (width 0.4) (layer "B.Cu") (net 3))
 (segment (start 110.3 112.7125) (end 109.2375 111.65) (width 0.4) (layer "B.Cu") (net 3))
 (segment (start 105.22 111.8325) (end 104.5 111.1125) (width 0.2) (layer "F.Cu") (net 5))
 (segment (start 105.15 106.2) (end 105.15 104.1) (width 0.2) (layer "F.Cu") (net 5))
 (segment (start 105.6 106.65) (end 105.15 106.2) (width 0.2) (layer "F.Cu") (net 5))
 (segment (start 104.5 111.1125) (end 104.675 111.1125) (width 0.4) (layer "F.Cu") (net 5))
 (segment (start 105.22 114.1) (end 105.22 111.8325) (width 0.2) (layer "F.Cu") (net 5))
 (via (at 105.6 106.65) (size 0.8) (drill 0.4) (layers "F.Cu" "B.Cu") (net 5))
 (segment (start 105.15 106.2) (end 105.15 104.1) (width 0.2) (layer "B.Cu") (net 5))
 (segment (start 105.6 106.65) (end 105.15 106.2) (width 0.2) (layer "B.Cu") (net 5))
 (segment (start 107.4 112.9) (end 107.8 112.5) (width 0.2) (layer "B.Cu") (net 5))
 (segment (start 107.35 107.35) (end 106.3 107.35) (width 0.2) (layer "B.Cu") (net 5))
 (segment (start 106.42 112.9) (end 107.4 112.9) (width 0.2) (layer "B.Cu") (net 5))
 (segment (start 106.3 107.35) (end 105.6 106.65) (width 0.2) (layer "B.Cu") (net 5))
 (segment (start 107.8 112.5) (end 107.8 107.8) (width 0.2) (layer "B.Cu") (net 5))
 (segment (start 107.8 107.8) (end 107.35 107.35) (width 0.2) (layer "B.Cu") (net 5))
 (segment (start 105.22 114.1) (end 106.42 112.9) (width 0.2) (layer "B.Cu") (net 5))
 (segment (start 106.65 106.65) (end 106.05 106.05) (width 0.2) (layer "F.Cu") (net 4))
 (segment (start 107 112.96) (end 107 111.1125) (width 0.2) (layer "F.Cu") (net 4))
 (segment (start 108.04 114) (end 107 112.96) (width 0.2) (layer "F.Cu") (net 4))
 (segment (start 106.05 106.05) (end 106.05 104.1) (width 0.2) (layer "F.Cu") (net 4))
 (segment (start 106.7 106.65) (end 106.65 106.65) (width 0.2) (layer "F.Cu") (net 4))
 (via (at 106.7 106.65) (size 0.8) (drill 0.4) (layers "F.Cu" "B.Cu") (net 4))
 (segment (start 106.05 106.05) (end 106.05 104.1) (width 0.2) (layer "B.Cu") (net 4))
 (segment (start 106.7 106.65) (end 107.218629 106.65) (width 0.2) (layer "B.Cu") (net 4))
 (segment (start 106.65 106.65) (end 106.05 106.05) (width 0.2) (layer "B.Cu") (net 4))
 (segment (start 108.1995 113.5605) (end 107.76 114) (width 0.2) (layer "B.Cu") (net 4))
 (segment (start 108.1995 113.8405) (end 108.04 114) (width 0.2) (layer "B.Cu") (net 4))
 (segment (start 107.218629 106.65) (end 108.2 107.631371) (width 0.2) (layer "B.Cu") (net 4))
 (segment (start 106.7 106.65) (end 106.65 106.65) (width 0.2) (layer "B.Cu") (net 4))
 (segment (start 108.2 113.66) (end 107.76 114.1) (width 0.2) (layer "B.Cu") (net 4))
 (segment (start 108.2 107.631371) (end 108.2 113.66) (width 0.2) (layer "B.Cu") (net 4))
 (segment (start 102 108.7875) (end 102 106.7) (width 0.4) (layer "F.Cu") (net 2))
 (segment (start 102.5 109.2875) (end 102 108.7875) (width 0.4) (layer "F.Cu") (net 2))
 (segment (start 102 106.5) (end 103.3 105.2) (width 0.4) (layer "F.Cu") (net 2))
 (segment (start 102 106.7) (end 102 106.5) (width 0.4) (layer "F.Cu") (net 2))
 (via (at 102 106.7) (size 0.8) (drill 0.4) (layers "F.Cu" "B.Cu") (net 2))
 (segment (start 102.05 106.65) (end 102.05 106.45) (width 0.4) (layer "B.Cu") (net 2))
 (segment (start 102.05 106.45) (end 103.35 105.15) (width 0.4) (layer "B.Cu") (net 2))
 (segment (start 103.15 106.7) (end 103.45 106.4) (width 0.2) (layer "F.Cu") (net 9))
 (segment (start 104.25 106.05) (end 104.25 104.1) (width 0.2) (layer "F.Cu") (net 9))
 (segment (start 103.45 106.4) (end 103.9 106.4) (width 0.2) (layer "F.Cu") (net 9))
 (segment (start 103.9 106.4) (end 104.25 106.05) (width 0.2) (layer "F.Cu") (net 9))
 (via (at 103.15 106.7) (size 0.8) (drill 0.4) (layers "F.Cu" "B.Cu") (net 9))
 (segment (start 102.9 108.75) (end 102.9 106.95) (width 0.2) (layer "B.Cu") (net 9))
 (segment (start 104.25 106.05) (end 104.25 104.1) (width 0.2) (layer "B.Cu") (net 9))
 (segment (start 103.9 106.4) (end 104.25 106.05) (width 0.2) (layer "B.Cu") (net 9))
 (segment (start 103.15 106.7) (end 103.45 106.4) (width 0.2) (layer "B.Cu") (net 9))
 (segment (start 103.45 106.4) (end 103.9 106.4) (width 0.2) (layer "B.Cu") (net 9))
 (segment (start 102.9 106.95) (end 103.15 106.7) (width 0.2) (layer "B.Cu") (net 9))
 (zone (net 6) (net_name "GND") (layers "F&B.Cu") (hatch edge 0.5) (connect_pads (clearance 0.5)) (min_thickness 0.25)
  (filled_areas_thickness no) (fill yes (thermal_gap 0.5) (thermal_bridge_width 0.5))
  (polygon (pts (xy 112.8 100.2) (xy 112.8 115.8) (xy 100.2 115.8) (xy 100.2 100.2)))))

